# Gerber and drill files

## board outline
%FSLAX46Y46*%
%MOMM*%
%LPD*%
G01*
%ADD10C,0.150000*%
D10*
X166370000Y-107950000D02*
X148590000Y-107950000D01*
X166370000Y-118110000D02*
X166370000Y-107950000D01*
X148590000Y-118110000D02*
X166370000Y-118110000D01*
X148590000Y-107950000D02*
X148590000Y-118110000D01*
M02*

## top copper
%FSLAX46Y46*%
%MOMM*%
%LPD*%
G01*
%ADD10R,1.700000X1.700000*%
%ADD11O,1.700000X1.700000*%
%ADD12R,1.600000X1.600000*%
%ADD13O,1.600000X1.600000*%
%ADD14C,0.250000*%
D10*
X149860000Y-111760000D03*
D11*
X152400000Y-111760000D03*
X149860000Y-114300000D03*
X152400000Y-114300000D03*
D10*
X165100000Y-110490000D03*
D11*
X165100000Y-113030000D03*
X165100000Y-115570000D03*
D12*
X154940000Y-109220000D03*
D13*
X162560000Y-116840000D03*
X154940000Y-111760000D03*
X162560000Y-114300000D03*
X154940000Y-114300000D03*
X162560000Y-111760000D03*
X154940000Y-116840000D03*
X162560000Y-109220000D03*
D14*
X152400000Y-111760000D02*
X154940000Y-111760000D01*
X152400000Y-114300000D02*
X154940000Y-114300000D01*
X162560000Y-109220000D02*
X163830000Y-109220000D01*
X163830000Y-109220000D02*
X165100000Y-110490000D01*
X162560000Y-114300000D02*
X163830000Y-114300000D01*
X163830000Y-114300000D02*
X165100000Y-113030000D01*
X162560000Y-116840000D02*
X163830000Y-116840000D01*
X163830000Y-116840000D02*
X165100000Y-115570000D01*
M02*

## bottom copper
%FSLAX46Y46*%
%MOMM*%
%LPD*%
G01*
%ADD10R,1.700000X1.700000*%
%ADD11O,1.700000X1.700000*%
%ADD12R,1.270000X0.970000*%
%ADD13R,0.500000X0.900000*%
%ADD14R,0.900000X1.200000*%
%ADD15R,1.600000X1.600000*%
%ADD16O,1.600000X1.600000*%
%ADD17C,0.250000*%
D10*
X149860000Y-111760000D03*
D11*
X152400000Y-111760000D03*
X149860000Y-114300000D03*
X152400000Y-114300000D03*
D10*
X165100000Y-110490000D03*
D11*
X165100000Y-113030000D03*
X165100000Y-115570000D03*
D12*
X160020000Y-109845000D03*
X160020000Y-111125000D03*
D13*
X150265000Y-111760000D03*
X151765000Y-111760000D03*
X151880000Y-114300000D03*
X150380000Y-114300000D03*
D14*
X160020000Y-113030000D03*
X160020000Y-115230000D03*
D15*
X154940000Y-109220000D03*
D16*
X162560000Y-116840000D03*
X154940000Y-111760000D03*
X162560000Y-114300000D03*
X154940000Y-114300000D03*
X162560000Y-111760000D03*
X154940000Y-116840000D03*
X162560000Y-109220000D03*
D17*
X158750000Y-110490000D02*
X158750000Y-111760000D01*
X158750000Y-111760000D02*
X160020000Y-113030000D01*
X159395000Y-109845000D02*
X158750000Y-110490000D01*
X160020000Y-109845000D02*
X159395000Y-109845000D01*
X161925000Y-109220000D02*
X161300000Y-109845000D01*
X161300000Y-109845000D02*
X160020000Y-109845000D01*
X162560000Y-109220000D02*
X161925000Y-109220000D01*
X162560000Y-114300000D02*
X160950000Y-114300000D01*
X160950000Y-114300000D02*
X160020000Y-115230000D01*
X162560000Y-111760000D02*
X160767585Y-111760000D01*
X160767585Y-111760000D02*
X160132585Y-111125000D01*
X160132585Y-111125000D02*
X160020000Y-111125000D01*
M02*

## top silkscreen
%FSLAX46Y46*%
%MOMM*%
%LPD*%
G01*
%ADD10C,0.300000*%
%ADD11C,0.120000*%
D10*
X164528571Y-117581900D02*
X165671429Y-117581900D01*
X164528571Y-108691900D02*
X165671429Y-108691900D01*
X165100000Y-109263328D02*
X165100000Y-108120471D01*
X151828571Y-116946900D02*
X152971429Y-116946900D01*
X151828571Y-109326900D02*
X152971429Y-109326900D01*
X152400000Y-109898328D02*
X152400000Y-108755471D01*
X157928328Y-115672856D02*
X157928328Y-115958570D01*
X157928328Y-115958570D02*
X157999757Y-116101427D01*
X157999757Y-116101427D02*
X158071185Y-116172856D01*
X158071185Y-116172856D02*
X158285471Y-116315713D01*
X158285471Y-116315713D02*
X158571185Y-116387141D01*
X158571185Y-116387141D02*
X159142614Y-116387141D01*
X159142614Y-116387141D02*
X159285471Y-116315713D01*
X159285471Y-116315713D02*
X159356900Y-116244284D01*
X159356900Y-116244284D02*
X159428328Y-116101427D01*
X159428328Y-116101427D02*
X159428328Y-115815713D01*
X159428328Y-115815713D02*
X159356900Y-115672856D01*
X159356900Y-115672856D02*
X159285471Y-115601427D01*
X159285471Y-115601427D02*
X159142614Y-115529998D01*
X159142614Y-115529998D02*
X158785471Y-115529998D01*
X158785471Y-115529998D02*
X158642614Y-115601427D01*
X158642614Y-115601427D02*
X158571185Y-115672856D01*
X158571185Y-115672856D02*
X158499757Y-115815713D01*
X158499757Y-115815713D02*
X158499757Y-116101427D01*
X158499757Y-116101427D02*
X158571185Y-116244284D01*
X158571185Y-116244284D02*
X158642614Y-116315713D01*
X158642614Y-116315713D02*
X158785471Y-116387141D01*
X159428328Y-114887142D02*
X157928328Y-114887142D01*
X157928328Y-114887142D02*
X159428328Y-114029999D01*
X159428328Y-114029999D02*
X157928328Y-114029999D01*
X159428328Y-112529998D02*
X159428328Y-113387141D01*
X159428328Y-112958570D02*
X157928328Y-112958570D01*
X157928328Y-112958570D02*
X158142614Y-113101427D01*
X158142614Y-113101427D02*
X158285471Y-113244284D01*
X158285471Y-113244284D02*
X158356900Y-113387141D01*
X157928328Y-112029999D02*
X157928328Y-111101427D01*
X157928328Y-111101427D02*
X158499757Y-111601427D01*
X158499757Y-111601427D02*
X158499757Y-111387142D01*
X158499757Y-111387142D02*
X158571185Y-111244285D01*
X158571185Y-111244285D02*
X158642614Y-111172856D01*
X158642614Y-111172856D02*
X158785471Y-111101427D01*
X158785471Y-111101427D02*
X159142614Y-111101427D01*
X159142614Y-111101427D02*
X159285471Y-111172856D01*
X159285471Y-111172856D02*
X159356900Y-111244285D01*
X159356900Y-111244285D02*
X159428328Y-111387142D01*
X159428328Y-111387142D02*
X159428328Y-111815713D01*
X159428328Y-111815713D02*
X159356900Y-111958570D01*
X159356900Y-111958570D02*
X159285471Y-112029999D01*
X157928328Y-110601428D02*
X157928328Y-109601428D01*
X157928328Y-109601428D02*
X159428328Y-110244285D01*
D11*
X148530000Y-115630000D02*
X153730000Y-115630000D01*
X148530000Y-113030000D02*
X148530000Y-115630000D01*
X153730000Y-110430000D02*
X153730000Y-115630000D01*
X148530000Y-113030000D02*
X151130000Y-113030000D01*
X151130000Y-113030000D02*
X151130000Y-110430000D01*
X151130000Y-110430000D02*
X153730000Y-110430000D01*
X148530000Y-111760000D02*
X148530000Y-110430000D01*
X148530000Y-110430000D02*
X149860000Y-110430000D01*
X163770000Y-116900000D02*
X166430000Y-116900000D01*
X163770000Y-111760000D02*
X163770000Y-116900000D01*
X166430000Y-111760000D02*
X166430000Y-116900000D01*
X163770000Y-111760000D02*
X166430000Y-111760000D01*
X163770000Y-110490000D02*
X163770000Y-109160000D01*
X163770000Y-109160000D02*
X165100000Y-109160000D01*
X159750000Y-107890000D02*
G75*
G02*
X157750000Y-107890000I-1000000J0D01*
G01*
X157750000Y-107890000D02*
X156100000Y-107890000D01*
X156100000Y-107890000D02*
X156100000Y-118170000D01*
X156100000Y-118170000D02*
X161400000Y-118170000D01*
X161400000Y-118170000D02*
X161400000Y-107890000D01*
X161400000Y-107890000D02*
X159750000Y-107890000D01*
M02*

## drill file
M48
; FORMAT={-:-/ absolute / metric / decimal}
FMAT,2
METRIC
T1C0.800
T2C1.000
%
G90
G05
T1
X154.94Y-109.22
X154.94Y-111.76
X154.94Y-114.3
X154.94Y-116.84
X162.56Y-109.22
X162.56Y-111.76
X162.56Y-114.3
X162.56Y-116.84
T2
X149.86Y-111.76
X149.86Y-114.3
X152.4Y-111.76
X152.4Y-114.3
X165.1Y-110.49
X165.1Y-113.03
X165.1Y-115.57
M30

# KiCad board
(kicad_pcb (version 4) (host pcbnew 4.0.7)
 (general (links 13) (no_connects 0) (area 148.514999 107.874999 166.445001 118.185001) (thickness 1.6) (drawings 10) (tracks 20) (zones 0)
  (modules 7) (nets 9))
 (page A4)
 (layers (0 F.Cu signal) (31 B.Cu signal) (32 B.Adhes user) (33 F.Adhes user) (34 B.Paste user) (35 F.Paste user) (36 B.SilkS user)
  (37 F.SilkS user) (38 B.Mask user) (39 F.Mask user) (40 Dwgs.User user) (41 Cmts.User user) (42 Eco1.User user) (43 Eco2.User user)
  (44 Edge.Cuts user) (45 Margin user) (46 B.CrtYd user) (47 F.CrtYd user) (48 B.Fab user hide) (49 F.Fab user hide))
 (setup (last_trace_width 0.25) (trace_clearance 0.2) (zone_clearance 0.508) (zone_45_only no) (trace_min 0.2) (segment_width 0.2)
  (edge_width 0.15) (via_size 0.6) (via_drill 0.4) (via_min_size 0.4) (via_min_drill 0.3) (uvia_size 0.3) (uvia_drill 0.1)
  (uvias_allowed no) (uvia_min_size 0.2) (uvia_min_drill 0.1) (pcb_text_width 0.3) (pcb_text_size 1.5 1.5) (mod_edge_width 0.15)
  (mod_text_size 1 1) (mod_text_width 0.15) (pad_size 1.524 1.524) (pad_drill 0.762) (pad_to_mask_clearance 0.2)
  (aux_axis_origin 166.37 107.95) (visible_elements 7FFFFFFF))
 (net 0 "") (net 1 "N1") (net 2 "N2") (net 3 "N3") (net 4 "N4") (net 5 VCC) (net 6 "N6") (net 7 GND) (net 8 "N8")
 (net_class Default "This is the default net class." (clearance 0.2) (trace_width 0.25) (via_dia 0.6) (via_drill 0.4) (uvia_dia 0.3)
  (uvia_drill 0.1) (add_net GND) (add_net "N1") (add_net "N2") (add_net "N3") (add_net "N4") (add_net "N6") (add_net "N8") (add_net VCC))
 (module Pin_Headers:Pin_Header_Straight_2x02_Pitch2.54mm (layer F.Cu) (at 149.86 111.76)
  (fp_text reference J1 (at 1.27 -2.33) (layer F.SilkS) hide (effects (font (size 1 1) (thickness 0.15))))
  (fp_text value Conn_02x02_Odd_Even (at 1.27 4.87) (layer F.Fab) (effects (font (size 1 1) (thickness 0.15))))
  (fp_line (start -1.33 3.87) (end 3.87 3.87) (layer F.SilkS) (width 0.12))
  (fp_line (start -1.33 1.27) (end -1.33 3.87) (layer F.SilkS) (width 0.12))
  (fp_line (start 3.87 -1.33) (end 3.87 3.87) (layer F.SilkS) (width 0.12))
  (fp_line (start -1.33 1.27) (end 1.27 1.27) (layer F.SilkS) (width 0.12))
  (fp_line (start 1.27 1.27) (end 1.27 -1.33) (layer F.SilkS) (width 0.12))
  (fp_line (start 1.27 -1.33) (end 3.87 -1.33) (layer F.SilkS) (width 0.12))
  (fp_line (start -1.33 0) (end -1.33 -1.33) (layer F.SilkS) (width 0.12))
  (fp_line (start -1.33 -1.33) (end 0 -1.33) (layer F.SilkS) (width 0.12))
  (pad 1 thru_hole rect (at 0 0) (size 1.7 1.7) (drill 1) (layers *.Cu *.Mask) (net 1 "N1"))
  (pad 2 thru_hole oval (at 2.54 0) (size 1.7 1.7) (drill 1) (layers *.Cu *.Mask) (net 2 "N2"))
  (pad 3 thru_hole oval (at 0 2.54) (size 1.7 1.7) (drill 1) (layers *.Cu *.Mask) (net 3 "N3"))
  (pad 4 thru_hole oval (at 2.54 2.54) (size 1.7 1.7) (drill 1) (layers *.Cu *.Mask) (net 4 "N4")))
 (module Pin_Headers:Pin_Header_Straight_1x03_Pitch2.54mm (layer F.Cu) (at 165.1 110.49)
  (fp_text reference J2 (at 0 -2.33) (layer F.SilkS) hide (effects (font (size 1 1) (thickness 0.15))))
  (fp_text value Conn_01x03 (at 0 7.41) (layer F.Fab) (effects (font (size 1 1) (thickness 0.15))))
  (fp_line (start -1.33 6.41) (end 1.33 6.41) (layer F.SilkS) (width 0.12))
  (fp_line (start -1.33 1.27) (end -1.33 6.41) (layer F.SilkS) (width 0.12))
  (fp_line (start 1.33 1.27) (end 1.33 6.41) (layer F.SilkS) (width 0.12))
  (fp_line (start -1.33 1.27) (end 1.33 1.27) (layer F.SilkS) (width 0.12))
  (fp_line (start -1.33 0) (end -1.33 -1.33) (layer F.SilkS) (width 0.12))
  (fp_line (start -1.33 -1.33) (end 0 -1.33) (layer F.SilkS) (width 0.12))
  (pad 1 thru_hole rect (at 0 0) (size 1.7 1.7) (drill 1) (layers *.Cu *.Mask) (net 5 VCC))
  (pad 2 thru_hole oval (at 0 2.54) (size 1.7 1.7) (drill 1) (layers *.Cu *.Mask) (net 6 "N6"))
  (pad 3 thru_hole oval (at 0 5.08) (size 1.7 1.7) (drill 1) (layers *.Cu *.Mask) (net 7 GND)))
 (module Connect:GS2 (layer B.Cu) (at 160.02 110.485 180)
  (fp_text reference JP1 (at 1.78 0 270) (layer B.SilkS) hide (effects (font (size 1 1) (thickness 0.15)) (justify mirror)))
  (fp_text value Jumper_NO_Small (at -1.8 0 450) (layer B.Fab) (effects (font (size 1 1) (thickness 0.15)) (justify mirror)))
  (pad 1 smd rect (at 0 0.64 180) (size 1.27 0.97) (layers B.Cu B.Paste B.Mask) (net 5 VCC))
  (pad 2 smd rect (at 0 -0.64 180) (size 1.27 0.97) (layers B.Cu B.Paste B.Mask) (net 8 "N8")))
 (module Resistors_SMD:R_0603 (layer B.Cu) (at 151.015 111.76)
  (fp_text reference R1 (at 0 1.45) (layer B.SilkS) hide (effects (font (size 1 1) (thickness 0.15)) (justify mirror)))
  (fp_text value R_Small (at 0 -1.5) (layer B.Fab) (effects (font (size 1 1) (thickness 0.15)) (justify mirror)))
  (pad 1 smd rect (at -0.75 0) (size 0.5 0.9) (layers B.Cu B.Paste B.Mask) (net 1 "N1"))
  (pad 2 smd rect (at 0.75 0) (size 0.5 0.9) (layers B.Cu B.Paste B.Mask) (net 2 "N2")))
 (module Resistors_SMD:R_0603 (layer B.Cu) (at 151.13 114.3 180)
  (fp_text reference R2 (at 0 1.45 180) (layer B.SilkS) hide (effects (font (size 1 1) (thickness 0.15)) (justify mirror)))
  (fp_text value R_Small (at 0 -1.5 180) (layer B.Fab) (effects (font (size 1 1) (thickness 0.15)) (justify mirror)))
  (pad 1 smd rect (at -0.75 0 180) (size 0.5 0.9) (layers B.Cu B.Paste B.Mask) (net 4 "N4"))
  (pad 2 smd rect (at 0.75 0 180) (size 0.5 0.9) (layers B.Cu B.Paste B.Mask) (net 3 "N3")))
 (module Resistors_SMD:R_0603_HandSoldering (layer B.Cu) (at 160.02 114.13 270)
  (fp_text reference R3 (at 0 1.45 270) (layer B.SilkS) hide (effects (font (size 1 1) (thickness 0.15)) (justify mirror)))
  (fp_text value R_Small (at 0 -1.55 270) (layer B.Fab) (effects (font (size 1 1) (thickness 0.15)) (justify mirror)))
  (pad 1 smd rect (at -1.1 0 270) (size 1.2 0.9) (layers B.Cu B.Paste B.Mask) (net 5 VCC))
  (pad 2 smd rect (at 1.1 0 270) (size 1.2 0.9) (layers B.Cu B.Paste B.Mask) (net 6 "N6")))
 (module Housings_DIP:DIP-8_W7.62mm (layer F.Cu) (at 154.94 109.22)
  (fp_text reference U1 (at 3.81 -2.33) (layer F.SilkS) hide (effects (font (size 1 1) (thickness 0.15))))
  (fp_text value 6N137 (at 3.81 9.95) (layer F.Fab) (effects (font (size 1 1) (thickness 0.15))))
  (fp_arc (start 3.81 -1.33) (end 2.81 -1.33) (angle -180) (layer F.SilkS) (width 0.12))
  (fp_line (start 2.81 -1.33) (end 1.16 -1.33) (layer F.SilkS) (width 0.12))
  (fp_line (start 1.16 -1.33) (end 1.16 8.95) (layer F.SilkS) (width 0.12))
  (fp_line (start 1.16 8.95) (end 6.46 8.95) (layer F.SilkS) (width 0.12))
  (fp_line (start 6.46 8.95) (end 6.46 -1.33) (layer F.SilkS) (width 0.12))
  (fp_line (start 6.46 -1.33) (end 4.81 -1.33) (layer F.SilkS) (width 0.12))
  (pad 1 thru_hole rect (at 0 0) (size 1.6 1.6) (drill 0.8) (layers *.Cu *.Mask))
  (pad 5 thru_hole oval (at 7.62 7.62) (size 1.6 1.6) (drill 0.8) (layers *.Cu *.Mask) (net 7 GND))
  (pad 2 thru_hole oval (at 0 2.54) (size 1.6 1.6) (drill 0.8) (layers *.Cu *.Mask) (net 2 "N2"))
  (pad 6 thru_hole oval (at 7.62 5.08) (size 1.6 1.6) (drill 0.8) (layers *.Cu *.Mask) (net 6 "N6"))
  (pad 3 thru_hole oval (at 0 5.08) (size 1.6 1.6) (drill 0.8) (layers *.Cu *.Mask) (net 4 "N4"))
  (pad 7 thru_hole oval (at 7.62 2.54) (size 1.6 1.6) (drill 0.8) (layers *.Cu *.Mask) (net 8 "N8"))
  (pad 4 thru_hole oval (at 0 7.62) (size 1.6 1.6) (drill 0.8) (layers *.Cu *.Mask))
  (pad 8 thru_hole oval (at 7.62 0) (size 1.6 1.6) (drill 0.8) (layers *.Cu *.Mask) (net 5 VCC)))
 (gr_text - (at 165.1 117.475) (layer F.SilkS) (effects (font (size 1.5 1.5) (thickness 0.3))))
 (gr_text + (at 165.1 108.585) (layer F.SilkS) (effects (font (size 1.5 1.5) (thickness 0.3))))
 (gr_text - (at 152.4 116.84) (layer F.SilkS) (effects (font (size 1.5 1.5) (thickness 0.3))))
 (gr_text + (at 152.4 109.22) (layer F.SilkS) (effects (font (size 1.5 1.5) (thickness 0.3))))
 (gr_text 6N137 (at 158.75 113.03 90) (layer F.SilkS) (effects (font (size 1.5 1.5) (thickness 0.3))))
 (gr_line (start 166.37 107.95) (end 148.59 107.95) (layer Edge.Cuts) (width 0.15))
 (gr_line (start 166.37 118.11) (end 166.37 107.95) (layer Edge.Cuts) (width 0.15))
 (gr_line (start 148.59 118.11) (end 166.37 118.11) (layer Edge.Cuts) (width 0.15))
 (gr_line (start 148.59 107.95) (end 148.59 118.11) (layer Edge.Cuts) (width 0.15))
 (segment (start 152.4 111.76) (end 154.94 111.76) (width 0.25) (layer F.Cu) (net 2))
 (segment (start 152.4 114.3) (end 154.94 114.3) (width 0.25) (layer F.Cu) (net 4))
 (segment (start 158.75 110.49) (end 158.75 111.76) (width 0.25) (layer B.Cu) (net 5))
 (segment (start 158.75 111.76) (end 160.02 113.03) (width 0.25) (layer B.Cu) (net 5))
 (segment (start 159.395 109.845) (end 158.75 110.49) (width 0.25) (layer B.Cu) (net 5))
 (segment (start 160.02 109.845) (end 159.395 109.845) (width 0.25) (layer B.Cu) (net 5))
 (segment (start 161.925 109.22) (end 161.3 109.845) (width 0.25) (layer B.Cu) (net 5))
 (segment (start 161.3 109.845) (end 160.02 109.845) (width 0.25) (layer B.Cu) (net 5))
 (segment (start 162.56 109.22) (end 161.925 109.22) (width 0.25) (layer B.Cu) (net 5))
 (segment (start 162.56 109.22) (end 163.83 109.22) (width 0.25) (layer F.Cu) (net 5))
 (segment (start 163.83 109.22) (end 165.1 110.49) (width 0.25) (layer F.Cu) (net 5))
 (segment (start 162.56 114.3) (end 160.95 114.3) (width 0.25) (layer B.Cu) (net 6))
 (segment (start 160.95 114.3) (end 160.02 115.23) (width 0.25) (layer B.Cu) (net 6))
 (segment (start 162.56 114.3) (end 163.83 114.3) (width 0.25) (layer F.Cu) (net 6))
 (segment (start 163.83 114.3) (end 165.1 113.03) (width 0.25) (layer F.Cu) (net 6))
 (segment (start 162.56 116.84) (end 163.83 116.84) (width 0.25) (layer F.Cu) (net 7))
 (segment (start 163.83 116.84) (end 165.1 115.57) (width 0.25) (layer F.Cu) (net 7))
 (segment (start 162.56 111.76) (end 160.767585 111.76) (width 0.25) (layer B.Cu) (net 8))
 (segment (start 160.767585 111.76) (end 160.132585 111.125) (width 0.25) (layer B.Cu) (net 8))
 (segment (start 160.132585 111.125) (end 160.02 111.125) (width 0.25) (layer B.Cu) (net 8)))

